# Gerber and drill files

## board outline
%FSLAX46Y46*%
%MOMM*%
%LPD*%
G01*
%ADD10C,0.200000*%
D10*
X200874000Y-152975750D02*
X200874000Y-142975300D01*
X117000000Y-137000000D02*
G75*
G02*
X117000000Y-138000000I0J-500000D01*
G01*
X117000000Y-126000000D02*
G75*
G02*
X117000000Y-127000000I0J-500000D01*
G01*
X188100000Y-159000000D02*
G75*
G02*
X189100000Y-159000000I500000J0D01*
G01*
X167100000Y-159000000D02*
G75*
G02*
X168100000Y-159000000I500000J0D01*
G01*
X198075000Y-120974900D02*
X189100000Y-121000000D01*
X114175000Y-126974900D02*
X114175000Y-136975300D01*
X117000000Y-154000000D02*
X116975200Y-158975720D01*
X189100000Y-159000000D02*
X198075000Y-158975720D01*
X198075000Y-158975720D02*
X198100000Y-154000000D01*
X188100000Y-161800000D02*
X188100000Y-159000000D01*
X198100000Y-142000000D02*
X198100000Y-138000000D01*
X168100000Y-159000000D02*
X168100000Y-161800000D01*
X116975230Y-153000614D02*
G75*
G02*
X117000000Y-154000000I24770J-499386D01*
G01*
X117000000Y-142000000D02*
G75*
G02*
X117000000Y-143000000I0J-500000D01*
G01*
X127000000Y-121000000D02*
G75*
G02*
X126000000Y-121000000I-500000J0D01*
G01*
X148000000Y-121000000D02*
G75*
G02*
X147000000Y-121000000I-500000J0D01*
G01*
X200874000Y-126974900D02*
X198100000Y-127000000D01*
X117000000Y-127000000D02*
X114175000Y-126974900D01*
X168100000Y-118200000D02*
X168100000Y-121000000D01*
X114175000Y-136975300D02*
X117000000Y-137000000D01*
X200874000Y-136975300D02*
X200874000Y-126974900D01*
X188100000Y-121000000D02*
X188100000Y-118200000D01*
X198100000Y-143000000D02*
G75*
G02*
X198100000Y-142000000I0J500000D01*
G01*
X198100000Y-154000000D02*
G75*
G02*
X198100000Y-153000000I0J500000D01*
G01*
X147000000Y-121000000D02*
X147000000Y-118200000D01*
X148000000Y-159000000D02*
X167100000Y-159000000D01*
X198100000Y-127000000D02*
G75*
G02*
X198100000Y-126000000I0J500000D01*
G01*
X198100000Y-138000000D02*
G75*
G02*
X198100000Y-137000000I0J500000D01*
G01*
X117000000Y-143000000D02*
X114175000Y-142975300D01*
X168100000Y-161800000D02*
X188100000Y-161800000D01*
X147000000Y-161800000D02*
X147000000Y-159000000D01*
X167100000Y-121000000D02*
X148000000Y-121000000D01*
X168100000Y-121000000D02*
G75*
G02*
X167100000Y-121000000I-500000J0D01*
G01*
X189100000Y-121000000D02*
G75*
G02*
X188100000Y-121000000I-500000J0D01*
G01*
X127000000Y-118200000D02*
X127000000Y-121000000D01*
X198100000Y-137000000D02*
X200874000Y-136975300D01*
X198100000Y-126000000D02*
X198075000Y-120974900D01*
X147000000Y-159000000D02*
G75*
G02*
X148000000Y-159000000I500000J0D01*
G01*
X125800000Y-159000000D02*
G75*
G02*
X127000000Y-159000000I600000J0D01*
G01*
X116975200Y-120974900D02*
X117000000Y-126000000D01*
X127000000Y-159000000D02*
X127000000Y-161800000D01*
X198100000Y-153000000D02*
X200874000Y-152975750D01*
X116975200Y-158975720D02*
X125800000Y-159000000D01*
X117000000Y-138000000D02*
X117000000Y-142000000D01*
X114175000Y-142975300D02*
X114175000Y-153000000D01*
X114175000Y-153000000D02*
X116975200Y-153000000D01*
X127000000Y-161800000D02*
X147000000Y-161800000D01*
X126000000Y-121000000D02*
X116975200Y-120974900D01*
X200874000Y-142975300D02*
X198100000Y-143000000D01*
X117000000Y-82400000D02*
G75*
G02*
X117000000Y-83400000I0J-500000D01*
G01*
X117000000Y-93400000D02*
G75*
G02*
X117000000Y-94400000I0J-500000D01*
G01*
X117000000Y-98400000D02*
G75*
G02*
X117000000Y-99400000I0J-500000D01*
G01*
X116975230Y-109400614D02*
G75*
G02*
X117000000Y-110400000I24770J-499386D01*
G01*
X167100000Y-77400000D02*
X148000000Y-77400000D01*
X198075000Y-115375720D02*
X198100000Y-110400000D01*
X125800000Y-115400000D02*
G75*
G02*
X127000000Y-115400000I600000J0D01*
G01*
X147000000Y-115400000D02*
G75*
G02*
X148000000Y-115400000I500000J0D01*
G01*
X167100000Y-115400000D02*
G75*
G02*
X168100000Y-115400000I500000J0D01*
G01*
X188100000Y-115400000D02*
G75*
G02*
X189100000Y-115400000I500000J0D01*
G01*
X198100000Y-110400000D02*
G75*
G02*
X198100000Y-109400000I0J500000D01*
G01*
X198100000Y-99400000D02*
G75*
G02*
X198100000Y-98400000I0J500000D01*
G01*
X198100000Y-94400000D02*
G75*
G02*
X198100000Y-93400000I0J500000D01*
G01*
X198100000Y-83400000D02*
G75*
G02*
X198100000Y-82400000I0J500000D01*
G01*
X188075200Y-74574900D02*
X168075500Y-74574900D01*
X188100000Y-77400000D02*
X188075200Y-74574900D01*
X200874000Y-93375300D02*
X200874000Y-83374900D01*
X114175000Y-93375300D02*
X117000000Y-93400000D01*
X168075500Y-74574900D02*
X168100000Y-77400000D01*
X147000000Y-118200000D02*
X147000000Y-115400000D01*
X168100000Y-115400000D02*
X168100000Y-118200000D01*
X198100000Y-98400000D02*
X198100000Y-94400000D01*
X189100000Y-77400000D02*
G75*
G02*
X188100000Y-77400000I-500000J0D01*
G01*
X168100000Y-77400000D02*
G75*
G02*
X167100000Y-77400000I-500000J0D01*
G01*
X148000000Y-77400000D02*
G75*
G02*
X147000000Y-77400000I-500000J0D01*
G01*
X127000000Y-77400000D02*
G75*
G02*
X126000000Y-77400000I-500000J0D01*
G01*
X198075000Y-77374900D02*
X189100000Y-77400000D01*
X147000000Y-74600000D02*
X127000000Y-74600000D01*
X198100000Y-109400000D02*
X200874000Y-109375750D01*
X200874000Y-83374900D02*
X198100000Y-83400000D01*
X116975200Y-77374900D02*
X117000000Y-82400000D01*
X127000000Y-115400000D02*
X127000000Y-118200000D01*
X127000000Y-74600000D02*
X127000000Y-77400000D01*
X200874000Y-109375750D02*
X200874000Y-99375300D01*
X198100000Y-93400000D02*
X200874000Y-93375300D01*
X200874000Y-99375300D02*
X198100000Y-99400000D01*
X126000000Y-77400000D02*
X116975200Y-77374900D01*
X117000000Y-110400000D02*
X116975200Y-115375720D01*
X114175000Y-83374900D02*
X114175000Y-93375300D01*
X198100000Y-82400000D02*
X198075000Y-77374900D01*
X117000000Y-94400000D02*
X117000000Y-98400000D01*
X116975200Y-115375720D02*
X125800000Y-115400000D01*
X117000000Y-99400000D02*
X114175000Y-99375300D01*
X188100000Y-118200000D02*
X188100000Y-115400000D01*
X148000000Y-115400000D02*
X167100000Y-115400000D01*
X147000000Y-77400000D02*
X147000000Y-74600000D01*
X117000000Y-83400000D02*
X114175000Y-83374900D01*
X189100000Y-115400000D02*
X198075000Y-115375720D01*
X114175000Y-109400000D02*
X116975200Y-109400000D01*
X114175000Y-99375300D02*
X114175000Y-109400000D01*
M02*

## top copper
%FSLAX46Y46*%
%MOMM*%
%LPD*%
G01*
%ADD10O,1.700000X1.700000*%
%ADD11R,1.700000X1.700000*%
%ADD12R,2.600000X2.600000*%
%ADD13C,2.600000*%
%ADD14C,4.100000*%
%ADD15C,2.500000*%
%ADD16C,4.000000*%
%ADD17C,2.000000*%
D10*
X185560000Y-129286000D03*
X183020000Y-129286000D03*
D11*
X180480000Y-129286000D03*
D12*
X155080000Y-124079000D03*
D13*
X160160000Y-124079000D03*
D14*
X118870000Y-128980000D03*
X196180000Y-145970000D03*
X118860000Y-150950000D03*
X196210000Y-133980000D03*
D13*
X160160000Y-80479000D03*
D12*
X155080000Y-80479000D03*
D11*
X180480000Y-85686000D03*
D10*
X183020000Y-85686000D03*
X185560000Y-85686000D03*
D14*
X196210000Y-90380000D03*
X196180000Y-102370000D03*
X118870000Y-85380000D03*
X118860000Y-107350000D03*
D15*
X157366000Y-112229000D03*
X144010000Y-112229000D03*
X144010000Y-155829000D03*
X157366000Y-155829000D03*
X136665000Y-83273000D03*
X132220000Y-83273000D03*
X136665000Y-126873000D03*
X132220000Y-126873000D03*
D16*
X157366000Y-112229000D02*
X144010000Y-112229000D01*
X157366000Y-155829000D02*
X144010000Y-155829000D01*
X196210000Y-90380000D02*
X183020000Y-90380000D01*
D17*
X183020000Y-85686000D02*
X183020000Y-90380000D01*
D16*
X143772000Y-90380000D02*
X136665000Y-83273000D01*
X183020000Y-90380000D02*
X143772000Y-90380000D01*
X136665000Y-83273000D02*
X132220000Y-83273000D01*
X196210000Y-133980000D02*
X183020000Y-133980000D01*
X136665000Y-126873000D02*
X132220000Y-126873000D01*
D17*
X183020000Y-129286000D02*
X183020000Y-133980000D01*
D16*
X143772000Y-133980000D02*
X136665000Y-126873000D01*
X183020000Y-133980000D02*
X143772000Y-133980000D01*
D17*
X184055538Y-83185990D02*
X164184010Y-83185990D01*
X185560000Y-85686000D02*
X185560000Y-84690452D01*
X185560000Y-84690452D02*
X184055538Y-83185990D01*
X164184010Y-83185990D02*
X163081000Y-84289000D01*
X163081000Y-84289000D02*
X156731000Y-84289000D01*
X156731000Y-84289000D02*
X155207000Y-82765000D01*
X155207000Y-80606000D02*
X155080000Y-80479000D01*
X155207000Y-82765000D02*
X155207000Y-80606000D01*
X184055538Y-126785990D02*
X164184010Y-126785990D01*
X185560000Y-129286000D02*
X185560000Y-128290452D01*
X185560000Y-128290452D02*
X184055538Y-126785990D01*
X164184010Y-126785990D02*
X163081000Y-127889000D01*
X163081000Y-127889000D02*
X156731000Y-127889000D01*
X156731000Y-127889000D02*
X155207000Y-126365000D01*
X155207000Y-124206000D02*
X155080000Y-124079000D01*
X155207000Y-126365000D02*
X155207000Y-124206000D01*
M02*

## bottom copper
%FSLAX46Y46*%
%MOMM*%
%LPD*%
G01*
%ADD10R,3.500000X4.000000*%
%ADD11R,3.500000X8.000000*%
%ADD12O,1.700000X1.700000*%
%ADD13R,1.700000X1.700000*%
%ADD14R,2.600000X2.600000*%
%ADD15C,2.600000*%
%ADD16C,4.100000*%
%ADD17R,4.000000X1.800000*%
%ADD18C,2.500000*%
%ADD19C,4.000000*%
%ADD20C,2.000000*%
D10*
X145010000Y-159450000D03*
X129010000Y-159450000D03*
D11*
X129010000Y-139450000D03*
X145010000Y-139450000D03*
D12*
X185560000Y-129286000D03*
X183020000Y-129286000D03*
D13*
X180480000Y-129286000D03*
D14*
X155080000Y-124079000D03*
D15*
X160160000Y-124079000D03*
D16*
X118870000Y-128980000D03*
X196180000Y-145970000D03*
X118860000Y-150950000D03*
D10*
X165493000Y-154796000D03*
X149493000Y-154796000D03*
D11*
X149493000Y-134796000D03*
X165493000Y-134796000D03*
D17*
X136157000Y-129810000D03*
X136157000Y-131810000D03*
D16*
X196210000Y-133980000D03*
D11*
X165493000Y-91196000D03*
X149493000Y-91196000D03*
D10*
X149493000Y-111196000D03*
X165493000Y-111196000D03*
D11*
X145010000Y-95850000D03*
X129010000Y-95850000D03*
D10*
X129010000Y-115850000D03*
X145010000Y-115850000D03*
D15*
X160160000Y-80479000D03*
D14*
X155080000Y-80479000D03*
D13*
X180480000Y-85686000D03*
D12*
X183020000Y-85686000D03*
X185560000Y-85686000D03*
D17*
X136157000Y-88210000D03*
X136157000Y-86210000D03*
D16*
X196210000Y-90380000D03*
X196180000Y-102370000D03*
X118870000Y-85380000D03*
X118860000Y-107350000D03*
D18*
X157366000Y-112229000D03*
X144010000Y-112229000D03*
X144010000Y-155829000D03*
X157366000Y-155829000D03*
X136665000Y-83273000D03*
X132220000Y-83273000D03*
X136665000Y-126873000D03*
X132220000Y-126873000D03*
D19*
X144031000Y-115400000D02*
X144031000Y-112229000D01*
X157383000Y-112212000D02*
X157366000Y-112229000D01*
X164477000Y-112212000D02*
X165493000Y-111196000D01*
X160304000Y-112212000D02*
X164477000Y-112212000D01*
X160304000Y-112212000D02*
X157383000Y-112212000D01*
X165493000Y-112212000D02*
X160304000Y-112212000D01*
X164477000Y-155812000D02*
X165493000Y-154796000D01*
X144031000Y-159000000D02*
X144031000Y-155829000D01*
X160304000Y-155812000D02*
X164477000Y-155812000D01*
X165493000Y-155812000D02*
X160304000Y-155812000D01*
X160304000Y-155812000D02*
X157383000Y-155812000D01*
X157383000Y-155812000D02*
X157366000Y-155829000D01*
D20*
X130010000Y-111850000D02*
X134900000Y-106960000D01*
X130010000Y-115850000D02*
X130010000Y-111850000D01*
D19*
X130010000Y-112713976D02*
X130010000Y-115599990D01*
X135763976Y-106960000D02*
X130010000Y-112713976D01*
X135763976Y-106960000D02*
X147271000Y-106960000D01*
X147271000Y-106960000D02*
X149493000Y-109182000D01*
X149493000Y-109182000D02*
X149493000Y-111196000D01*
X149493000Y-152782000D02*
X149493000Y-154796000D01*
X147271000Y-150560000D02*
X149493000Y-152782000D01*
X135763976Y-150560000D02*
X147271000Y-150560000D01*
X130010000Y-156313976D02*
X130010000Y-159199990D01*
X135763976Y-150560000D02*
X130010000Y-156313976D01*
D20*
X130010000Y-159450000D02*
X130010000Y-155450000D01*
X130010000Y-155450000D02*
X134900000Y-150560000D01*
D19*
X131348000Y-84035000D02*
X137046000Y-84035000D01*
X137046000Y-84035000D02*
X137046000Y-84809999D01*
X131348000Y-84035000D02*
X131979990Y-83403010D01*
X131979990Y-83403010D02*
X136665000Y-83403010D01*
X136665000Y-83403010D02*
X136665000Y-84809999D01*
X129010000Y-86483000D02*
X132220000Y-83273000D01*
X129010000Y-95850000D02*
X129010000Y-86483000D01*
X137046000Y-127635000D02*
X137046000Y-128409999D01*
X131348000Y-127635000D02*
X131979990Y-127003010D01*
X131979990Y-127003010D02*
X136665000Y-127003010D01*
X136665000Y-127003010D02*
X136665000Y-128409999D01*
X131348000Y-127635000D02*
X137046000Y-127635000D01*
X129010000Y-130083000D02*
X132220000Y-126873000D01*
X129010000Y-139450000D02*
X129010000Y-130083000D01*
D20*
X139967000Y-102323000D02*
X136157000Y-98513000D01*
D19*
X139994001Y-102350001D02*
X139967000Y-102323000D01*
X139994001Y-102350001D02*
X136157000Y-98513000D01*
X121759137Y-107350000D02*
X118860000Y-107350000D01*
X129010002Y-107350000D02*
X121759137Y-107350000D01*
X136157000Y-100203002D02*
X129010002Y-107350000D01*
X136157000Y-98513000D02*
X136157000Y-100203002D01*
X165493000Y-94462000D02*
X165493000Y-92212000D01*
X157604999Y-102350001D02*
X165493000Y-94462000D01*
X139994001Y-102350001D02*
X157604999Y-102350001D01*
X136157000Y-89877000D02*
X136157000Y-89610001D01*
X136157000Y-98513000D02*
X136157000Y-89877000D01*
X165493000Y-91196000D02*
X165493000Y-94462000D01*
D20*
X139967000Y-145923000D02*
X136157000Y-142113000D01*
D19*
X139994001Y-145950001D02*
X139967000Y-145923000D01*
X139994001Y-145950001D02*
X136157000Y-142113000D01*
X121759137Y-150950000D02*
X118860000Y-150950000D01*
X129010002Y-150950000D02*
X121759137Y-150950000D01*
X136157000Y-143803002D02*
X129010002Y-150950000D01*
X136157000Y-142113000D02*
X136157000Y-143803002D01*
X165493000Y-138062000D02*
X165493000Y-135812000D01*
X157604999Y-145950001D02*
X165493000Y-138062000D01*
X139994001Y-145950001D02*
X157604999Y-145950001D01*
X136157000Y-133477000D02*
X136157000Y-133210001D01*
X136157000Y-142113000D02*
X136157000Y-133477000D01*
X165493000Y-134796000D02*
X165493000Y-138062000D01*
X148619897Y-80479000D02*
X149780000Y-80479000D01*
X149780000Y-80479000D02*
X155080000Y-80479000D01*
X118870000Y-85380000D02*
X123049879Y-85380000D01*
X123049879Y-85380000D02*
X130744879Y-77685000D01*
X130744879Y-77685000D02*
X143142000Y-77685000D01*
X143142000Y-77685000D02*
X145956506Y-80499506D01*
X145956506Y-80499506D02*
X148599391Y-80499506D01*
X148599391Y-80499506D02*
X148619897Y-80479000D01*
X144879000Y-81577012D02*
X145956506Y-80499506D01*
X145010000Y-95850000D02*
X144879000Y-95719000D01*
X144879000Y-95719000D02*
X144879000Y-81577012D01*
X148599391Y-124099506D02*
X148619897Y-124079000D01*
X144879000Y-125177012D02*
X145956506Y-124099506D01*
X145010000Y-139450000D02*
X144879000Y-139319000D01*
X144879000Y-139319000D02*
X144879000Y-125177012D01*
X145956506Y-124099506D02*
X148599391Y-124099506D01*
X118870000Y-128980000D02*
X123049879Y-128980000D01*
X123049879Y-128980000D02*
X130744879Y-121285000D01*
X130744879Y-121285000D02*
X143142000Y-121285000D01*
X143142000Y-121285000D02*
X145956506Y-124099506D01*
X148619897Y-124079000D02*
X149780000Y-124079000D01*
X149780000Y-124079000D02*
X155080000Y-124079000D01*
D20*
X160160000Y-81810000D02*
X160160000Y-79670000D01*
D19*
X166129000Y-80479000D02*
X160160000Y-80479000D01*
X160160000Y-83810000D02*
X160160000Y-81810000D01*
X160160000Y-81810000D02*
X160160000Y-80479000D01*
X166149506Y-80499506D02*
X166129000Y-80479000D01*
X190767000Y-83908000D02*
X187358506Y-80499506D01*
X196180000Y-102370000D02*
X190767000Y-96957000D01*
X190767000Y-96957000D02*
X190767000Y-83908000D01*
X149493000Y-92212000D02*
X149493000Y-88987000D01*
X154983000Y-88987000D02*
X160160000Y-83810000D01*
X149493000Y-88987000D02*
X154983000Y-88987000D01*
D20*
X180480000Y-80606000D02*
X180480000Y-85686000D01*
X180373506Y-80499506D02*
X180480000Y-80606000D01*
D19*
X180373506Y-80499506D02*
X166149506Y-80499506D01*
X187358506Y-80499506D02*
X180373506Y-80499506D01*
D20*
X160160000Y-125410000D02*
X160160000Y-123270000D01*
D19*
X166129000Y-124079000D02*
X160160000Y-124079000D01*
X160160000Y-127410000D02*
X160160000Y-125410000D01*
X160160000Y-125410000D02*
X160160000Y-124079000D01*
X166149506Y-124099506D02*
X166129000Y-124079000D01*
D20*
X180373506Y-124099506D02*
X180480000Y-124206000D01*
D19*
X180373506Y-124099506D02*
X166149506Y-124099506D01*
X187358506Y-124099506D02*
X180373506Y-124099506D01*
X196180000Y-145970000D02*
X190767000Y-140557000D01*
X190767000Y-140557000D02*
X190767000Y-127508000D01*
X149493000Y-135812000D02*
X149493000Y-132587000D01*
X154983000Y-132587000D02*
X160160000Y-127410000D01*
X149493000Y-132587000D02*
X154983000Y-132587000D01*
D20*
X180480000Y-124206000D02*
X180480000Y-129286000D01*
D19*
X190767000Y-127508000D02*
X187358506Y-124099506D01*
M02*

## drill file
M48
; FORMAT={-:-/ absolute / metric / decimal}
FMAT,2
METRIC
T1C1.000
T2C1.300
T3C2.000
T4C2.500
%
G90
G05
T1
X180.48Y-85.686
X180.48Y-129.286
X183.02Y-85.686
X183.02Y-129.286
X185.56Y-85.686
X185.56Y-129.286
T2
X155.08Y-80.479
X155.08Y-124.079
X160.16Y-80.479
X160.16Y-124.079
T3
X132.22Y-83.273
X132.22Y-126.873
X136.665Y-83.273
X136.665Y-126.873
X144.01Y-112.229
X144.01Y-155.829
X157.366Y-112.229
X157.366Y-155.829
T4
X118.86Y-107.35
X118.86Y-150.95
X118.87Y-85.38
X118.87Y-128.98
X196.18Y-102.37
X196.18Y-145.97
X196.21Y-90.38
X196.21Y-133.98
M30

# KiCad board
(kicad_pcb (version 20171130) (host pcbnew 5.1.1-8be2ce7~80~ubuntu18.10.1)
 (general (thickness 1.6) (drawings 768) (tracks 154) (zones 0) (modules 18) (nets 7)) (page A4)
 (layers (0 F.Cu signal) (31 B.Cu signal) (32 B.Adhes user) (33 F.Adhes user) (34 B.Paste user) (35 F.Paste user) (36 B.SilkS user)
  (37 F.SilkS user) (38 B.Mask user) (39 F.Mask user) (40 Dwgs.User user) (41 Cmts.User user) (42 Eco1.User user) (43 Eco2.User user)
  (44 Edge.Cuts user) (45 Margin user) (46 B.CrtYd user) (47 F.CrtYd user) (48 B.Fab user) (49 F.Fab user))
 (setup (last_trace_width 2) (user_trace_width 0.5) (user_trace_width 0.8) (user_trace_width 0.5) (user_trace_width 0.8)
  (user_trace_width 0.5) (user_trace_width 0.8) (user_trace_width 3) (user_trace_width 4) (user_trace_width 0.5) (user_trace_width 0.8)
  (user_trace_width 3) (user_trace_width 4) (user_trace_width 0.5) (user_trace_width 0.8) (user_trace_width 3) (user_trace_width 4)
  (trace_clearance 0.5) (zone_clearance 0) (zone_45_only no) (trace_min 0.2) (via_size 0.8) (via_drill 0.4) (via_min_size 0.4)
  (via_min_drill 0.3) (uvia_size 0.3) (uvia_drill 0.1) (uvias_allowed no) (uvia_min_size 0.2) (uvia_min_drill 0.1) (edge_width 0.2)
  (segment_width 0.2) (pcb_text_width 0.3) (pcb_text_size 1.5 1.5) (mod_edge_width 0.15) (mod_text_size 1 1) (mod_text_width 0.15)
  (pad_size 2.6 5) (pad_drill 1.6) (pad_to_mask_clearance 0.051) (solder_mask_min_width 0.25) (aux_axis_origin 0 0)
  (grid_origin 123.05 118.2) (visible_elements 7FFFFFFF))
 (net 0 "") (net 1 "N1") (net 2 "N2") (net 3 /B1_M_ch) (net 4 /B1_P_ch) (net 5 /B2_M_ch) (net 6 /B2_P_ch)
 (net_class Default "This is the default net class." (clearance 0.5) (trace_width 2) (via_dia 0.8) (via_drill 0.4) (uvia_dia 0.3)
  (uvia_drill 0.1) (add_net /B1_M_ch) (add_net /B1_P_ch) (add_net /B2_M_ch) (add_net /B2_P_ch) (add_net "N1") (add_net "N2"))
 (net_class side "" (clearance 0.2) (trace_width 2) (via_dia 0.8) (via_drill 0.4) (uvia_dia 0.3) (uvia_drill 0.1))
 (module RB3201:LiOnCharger (layer B.Cu) (at 137.01 150.45)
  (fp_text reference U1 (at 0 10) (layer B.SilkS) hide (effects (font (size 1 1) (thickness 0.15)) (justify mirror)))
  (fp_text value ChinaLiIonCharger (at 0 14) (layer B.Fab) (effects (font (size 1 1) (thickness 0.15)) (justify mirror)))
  (pad 1 smd rect (at 8 9) (size 3.5 4) (layers B.Cu B.Paste B.Mask) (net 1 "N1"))
  (pad 2 smd rect (at -8 9) (size 3.5 4) (layers B.Cu B.Paste B.Mask) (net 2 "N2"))
  (pad 3 smd rect (at -8 -11) (size 3.5 8) (layers B.Cu B.Paste B.Mask) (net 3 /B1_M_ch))
  (pad 4 smd rect (at 8 -11) (size 3.5 8) (layers B.Cu B.Paste B.Mask) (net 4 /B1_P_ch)))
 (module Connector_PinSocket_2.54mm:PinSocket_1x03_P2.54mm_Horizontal (layer B.Cu) (at 180.48 129.286 270)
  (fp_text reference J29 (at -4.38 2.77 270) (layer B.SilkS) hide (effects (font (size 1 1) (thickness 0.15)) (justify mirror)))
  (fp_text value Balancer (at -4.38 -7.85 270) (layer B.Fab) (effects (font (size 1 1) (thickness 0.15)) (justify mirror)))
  (pad 3 thru_hole oval (at 0 -5.08 270) (size 1.7 1.7) (drill 1) (layers *.Cu *.Mask) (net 4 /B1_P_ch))
  (pad 2 thru_hole oval (at 0 -2.54 270) (size 1.7 1.7) (drill 1) (layers *.Cu *.Mask) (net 3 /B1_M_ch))
  (pad 1 thru_hole rect (at 0 0 270) (size 1.7 1.7) (drill 1) (layers *.Cu *.Mask) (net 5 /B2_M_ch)))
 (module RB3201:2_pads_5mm (layer B.Cu) (at 155.08 124.079)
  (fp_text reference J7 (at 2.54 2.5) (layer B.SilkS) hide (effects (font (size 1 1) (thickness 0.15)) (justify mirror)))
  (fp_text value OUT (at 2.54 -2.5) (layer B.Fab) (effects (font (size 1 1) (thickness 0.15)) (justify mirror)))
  (pad 1 thru_hole rect (at 0 0) (size 2.6 2.6) (drill 1.3) (layers *.Cu *.Mask) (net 4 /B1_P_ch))
  (pad 2 thru_hole circle (at 5.08 0) (size 2.6 2.6) (drill 1.3) (layers *.Cu *.Mask) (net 5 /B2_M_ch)))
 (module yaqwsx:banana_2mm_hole (layer F.Cu) (at 118.87 128.98)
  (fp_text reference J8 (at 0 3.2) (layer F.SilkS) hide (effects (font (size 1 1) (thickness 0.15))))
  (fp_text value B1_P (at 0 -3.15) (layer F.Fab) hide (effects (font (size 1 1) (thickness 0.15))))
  (pad 1 thru_hole circle (at 0 0) (size 4.1 4.1) (drill 2.5) (layers *.Cu *.Mask) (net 4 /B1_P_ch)))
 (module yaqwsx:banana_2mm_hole (layer F.Cu) (at 196.18 145.97)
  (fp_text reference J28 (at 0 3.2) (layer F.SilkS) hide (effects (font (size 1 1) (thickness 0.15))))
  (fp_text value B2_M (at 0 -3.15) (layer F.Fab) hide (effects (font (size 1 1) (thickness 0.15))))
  (pad 1 thru_hole circle (at 0 0) (size 4.1 4.1) (drill 2.5) (layers *.Cu *.Mask) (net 5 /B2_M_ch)))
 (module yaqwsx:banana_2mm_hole (layer F.Cu) (at 118.86 150.95)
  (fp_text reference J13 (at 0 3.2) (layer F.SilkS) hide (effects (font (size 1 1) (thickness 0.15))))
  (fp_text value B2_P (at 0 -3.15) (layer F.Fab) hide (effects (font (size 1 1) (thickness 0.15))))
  (pad 1 thru_hole circle (at 0 0) (size 4.1 4.1) (drill 2.5) (layers *.Cu *.Mask) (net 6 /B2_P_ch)))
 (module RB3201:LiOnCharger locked (layer B.Cu) (at 157.493 145.796)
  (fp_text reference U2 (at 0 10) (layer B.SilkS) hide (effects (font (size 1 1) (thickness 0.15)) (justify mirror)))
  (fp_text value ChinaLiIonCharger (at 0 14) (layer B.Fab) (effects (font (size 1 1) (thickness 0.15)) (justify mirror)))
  (pad 1 smd rect (at 8 9) (size 3.5 4) (layers B.Cu B.Paste B.Mask) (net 1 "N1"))
  (pad 2 smd rect (at -8 9) (size 3.5 4) (layers B.Cu B.Paste B.Mask) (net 2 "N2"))
  (pad 3 smd rect (at -8 -11) (size 3.5 8) (layers B.Cu B.Paste B.Mask) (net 5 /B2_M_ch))
  (pad 4 smd rect (at 8 -11) (size 3.5 8) (layers B.Cu B.Paste B.Mask) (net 6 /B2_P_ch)))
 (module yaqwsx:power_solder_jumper (layer B.Cu) (at 136.157 130.81 270)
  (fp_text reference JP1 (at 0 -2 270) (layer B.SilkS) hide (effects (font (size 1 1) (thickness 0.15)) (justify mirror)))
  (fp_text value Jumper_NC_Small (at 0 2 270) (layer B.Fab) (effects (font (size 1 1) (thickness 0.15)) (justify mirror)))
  (pad 1 smd rect (at -1 0 270) (size 1.8 4) (layers B.Cu B.Paste B.Mask) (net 3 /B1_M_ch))
  (pad 2 smd rect (at 1 0 270) (size 1.8 4) (layers B.Cu B.Paste B.Mask) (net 6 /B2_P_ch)))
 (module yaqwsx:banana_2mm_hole (layer F.Cu) (at 196.21 133.98)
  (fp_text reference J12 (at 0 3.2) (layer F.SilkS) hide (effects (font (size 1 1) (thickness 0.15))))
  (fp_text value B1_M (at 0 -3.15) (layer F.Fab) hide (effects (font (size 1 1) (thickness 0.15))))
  (pad 1 thru_hole circle (at 0 0) (size 4.1 4.1) (drill 2.5) (layers *.Cu *.Mask) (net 3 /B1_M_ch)))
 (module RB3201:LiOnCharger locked (layer B.Cu) (at 157.493 102.196)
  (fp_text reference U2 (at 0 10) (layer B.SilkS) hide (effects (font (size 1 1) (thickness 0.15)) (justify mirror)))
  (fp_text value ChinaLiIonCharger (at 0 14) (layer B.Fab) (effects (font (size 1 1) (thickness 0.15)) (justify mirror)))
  (pad 4 smd rect (at 8 -11) (size 3.5 8) (layers B.Cu B.Paste B.Mask) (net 6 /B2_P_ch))
  (pad 3 smd rect (at -8 -11) (size 3.5 8) (layers B.Cu B.Paste B.Mask) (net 5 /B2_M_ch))
  (pad 2 smd rect (at -8 9) (size 3.5 4) (layers B.Cu B.Paste B.Mask) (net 2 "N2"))
  (pad 1 smd rect (at 8 9) (size 3.5 4) (layers B.Cu B.Paste B.Mask) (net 1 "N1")))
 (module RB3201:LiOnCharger (layer B.Cu) (at 137.01 106.85)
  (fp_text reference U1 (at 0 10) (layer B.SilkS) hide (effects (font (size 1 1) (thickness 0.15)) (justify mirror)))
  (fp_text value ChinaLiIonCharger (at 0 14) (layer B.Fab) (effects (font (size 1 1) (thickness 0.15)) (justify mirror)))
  (pad 4 smd rect (at 8 -11) (size 3.5 8) (layers B.Cu B.Paste B.Mask) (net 4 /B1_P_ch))
  (pad 3 smd rect (at -8 -11) (size 3.5 8) (layers B.Cu B.Paste B.Mask) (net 3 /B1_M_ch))
  (pad 2 smd rect (at -8 9) (size 3.5 4) (layers B.Cu B.Paste B.Mask) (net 2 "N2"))
  (pad 1 smd rect (at 8 9) (size 3.5 4) (layers B.Cu B.Paste B.Mask) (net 1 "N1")))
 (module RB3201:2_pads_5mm (layer B.Cu) (at 155.08 80.479)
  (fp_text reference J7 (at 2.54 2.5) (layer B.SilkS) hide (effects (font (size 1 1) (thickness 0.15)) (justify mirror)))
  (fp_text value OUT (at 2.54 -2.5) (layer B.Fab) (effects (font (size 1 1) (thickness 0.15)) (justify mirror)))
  (pad 2 thru_hole circle (at 5.08 0) (size 2.6 2.6) (drill 1.3) (layers *.Cu *.Mask) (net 5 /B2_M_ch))
  (pad 1 thru_hole rect (at 0 0) (size 2.6 2.6) (drill 1.3) (layers *.Cu *.Mask) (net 4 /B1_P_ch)))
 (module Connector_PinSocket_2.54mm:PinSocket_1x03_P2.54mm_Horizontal (layer B.Cu) (at 180.48 85.686 270)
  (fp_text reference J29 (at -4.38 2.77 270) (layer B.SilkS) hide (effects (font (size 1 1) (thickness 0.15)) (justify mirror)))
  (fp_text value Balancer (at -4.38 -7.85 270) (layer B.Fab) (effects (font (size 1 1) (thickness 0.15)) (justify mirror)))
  (pad 1 thru_hole rect (at 0 0 270) (size 1.7 1.7) (drill 1) (layers *.Cu *.Mask) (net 5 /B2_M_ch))
  (pad 2 thru_hole oval (at 0 -2.54 270) (size 1.7 1.7) (drill 1) (layers *.Cu *.Mask) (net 3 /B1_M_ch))
  (pad 3 thru_hole oval (at 0 -5.08 270) (size 1.7 1.7) (drill 1) (layers *.Cu *.Mask) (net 4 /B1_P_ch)))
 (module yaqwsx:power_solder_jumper (layer B.Cu) (at 136.157 87.21 270)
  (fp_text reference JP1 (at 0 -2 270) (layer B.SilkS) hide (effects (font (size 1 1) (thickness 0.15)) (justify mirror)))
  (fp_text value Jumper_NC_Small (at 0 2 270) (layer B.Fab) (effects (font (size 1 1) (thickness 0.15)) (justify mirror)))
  (pad 2 smd rect (at 1 0 270) (size 1.8 4) (layers B.Cu B.Paste B.Mask) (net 6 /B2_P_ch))
  (pad 1 smd rect (at -1 0 270) (size 1.8 4) (layers B.Cu B.Paste B.Mask) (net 3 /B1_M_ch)))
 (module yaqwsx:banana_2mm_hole (layer F.Cu) (at 196.21 90.38)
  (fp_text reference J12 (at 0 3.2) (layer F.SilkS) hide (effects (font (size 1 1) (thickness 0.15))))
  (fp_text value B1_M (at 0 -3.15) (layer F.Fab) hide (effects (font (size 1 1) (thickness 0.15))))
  (pad 1 thru_hole circle (at 0 0) (size 4.1 4.1) (drill 2.5) (layers *.Cu *.Mask) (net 3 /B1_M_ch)))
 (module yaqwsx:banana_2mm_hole (layer F.Cu) (at 196.18 102.37)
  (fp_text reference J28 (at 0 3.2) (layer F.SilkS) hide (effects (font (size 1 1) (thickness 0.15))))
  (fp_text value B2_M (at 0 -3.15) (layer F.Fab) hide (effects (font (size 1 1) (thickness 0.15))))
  (pad 1 thru_hole circle (at 0 0) (size 4.1 4.1) (drill 2.5) (layers *.Cu *.Mask) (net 5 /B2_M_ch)))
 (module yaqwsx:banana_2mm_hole (layer F.Cu) (at 118.87 85.38)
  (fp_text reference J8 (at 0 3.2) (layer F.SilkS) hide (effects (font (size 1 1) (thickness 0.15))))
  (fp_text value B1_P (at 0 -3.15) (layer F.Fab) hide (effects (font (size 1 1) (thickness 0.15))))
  (pad 1 thru_hole circle (at 0 0) (size 4.1 4.1) (drill 2.5) (layers *.Cu *.Mask) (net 4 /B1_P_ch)))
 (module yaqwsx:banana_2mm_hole (layer F.Cu) (at 118.86 107.35)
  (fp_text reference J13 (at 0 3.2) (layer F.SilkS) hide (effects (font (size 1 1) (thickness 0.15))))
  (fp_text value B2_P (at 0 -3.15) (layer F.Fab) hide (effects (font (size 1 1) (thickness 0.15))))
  (pad 1 thru_hole circle (at 0 0) (size 4.1 4.1) (drill 2.5) (layers *.Cu *.Mask) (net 6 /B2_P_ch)))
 (gr_line (start 200.874 152.97575) (end 200.874 142.9753) (layer Edge.Cuts) (width 0.2))
 (gr_arc (start 117 137.5) (end 117 138) (angle -180) (layer Edge.Cuts) (width 0.2))
 (gr_arc (start 117 126.5) (end 117 127) (angle -180) (layer Edge.Cuts) (width 0.2))
 (gr_arc (start 188.6 159) (end 189.1 159) (angle -180) (layer Edge.Cuts) (width 0.2))
 (gr_arc (start 167.6 159) (end 168.1 159) (angle -180) (layer Edge.Cuts) (width 0.2))
 (gr_line (start 198.075 120.9749) (end 189.1 121) (layer Edge.Cuts) (width 0.2))
 (gr_line (start 114.175 126.9749) (end 114.175 136.9753) (layer Edge.Cuts) (width 0.2))
 (gr_line (start 117 154) (end 116.9752 158.97572) (layer Edge.Cuts) (width 0.2))
 (gr_line (start 189.1 159) (end 198.075 158.97572) (layer Edge.Cuts) (width 0.2))
 (gr_line (start 198.075 158.97572) (end 198.1 154) (layer Edge.Cuts) (width 0.2))
 (gr_line (start 188.1 161.8) (end 188.1 159) (layer Edge.Cuts) (width 0.2))
 (gr_line (start 198.1 142) (end 198.1 138) (layer Edge.Cuts) (width 0.2))
 (gr_line (start 168.1 159) (end 168.1 161.8) (layer Edge.Cuts) (width 0.2))
 (gr_arc (start 117 153.5) (end 117 154) (angle -182.8395436) (layer Edge.Cuts) (width 0.2))
 (gr_arc (start 117 142.5) (end 117 143) (angle -180) (layer Edge.Cuts) (width 0.2))
 (gr_arc (start 126.5 121) (end 126 121) (angle -180) (layer Edge.Cuts) (width 0.2))
 (gr_arc (start 147.5 121) (end 147 121) (angle -180) (layer Edge.Cuts) (width 0.2))
 (gr_line (start 200.874 126.9749) (end 198.1 127) (layer Edge.Cuts) (width 0.2))
 (gr_line (start 117 127) (end 114.175 126.9749) (layer Edge.Cuts) (width 0.2))
 (gr_line (start 168.1 118.2) (end 168.1 121) (layer Edge.Cuts) (width 0.2))
 (gr_line (start 114.175 136.9753) (end 117 137) (layer Edge.Cuts) (width 0.2))
 (gr_line (start 200.874 136.9753) (end 200.874 126.9749) (layer Edge.Cuts) (width 0.2))
 (gr_line (start 188.1 121) (end 188.1 118.2) (layer Edge.Cuts) (width 0.2))
 (gr_arc (start 198.1 142.5) (end 198.1 142) (angle -180) (layer Edge.Cuts) (width 0.2))
 (gr_arc (start 198.1 153.5) (end 198.1 153) (angle -180) (layer Edge.Cuts) (width 0.2))
 (gr_line (start 147 121) (end 147 118.2) (layer Edge.Cuts) (width 0.2))
 (gr_line (start 148 159) (end 167.1 159) (layer Edge.Cuts) (width 0.2))
 (gr_arc (start 198.1 126.5) (end 198.1 126) (angle -180) (layer Edge.Cuts) (width 0.2))
 (gr_arc (start 198.1 137.5) (end 198.1 137) (angle -180) (layer Edge.Cuts) (width 0.2))
 (gr_line (start 117 143) (end 114.175 142.9753) (layer Edge.Cuts) (width 0.2))
 (gr_line (start 168.1 161.8) (end 188.1 161.8) (layer Edge.Cuts) (width 0.2))
 (gr_line (start 147 161.8) (end 147 159) (layer Edge.Cuts) (width 0.2))
 (gr_line (start 167.1 121) (end 148 121) (layer Edge.Cuts) (width 0.2))
 (gr_arc (start 167.6 121) (end 167.1 121) (angle -180) (layer Edge.Cuts) (width 0.2))
 (gr_arc (start 188.6 121) (end 188.1 121) (angle -180) (layer Edge.Cuts) (width 0.2))
 (gr_line (start 127 118.2) (end 127 121) (layer Edge.Cuts) (width 0.2))
 (gr_line (start 198.1 137) (end 200.874 136.9753) (layer Edge.Cuts) (width 0.2))
 (gr_line (start 198.1 126) (end 198.075 120.9749) (layer Edge.Cuts) (width 0.2))
 (gr_arc (start 147.5 159) (end 148 159) (angle -180) (layer Edge.Cuts) (width 0.2))
 (gr_arc (start 126.4 159) (end 127 159) (angle -180) (layer Edge.Cuts) (width 0.2))
 (gr_line (start 116.9752 120.9749) (end 117 126) (layer Edge.Cuts) (width 0.2))
 (gr_line (start 127 159) (end 127 161.8) (layer Edge.Cuts) (width 0.2))
 (gr_line (start 198.1 153) (end 200.874 152.97575) (layer Edge.Cuts) (width 0.2))
 (gr_line (start 116.9752 158.97572) (end 125.8 159) (layer Edge.Cuts) (width 0.2))
 (gr_line (start 117 138) (end 117 142) (layer Edge.Cuts) (width 0.2))
 (gr_line (start 114.175 142.9753) (end 114.175 153) (layer Edge.Cuts) (width 0.2))
 (gr_line (start 114.175 153) (end 116.9752 153) (layer Edge.Cuts) (width 0.2))
 (gr_line (start 127 161.8) (end 147 161.8) (layer Edge.Cuts) (width 0.2))
 (gr_line (start 126 121) (end 116.9752 120.9749) (layer Edge.Cuts) (width 0.2))
 (gr_line (start 200.874 142.9753) (end 198.1 143) (layer Edge.Cuts) (width 0.2))
 (gr_arc (start 117 82.9) (end 117 83.4) (angle -180) (layer Edge.Cuts) (width 0.2))
 (gr_arc (start 117 93.9) (end 117 94.4) (angle -180) (layer Edge.Cuts) (width 0.2))
 (gr_arc (start 117 98.9) (end 117 99.4) (angle -180) (layer Edge.Cuts) (width 0.2))
 (gr_arc (start 117 109.9) (end 117 110.4) (angle -182.8395436) (layer Edge.Cuts) (width 0.2))
 (gr_line (start 167.1 77.4) (end 148 77.4) (layer Edge.Cuts) (width 0.2))
 (gr_line (start 198.075 115.37572) (end 198.1 110.4) (layer Edge.Cuts) (width 0.2))
 (gr_arc (start 126.4 115.4) (end 127 115.4) (angle -180) (layer Edge.Cuts) (width 0.2))
 (gr_arc (start 147.5 115.4) (end 148 115.4) (angle -180) (layer Edge.Cuts) (width 0.2))
 (gr_arc (start 167.6 115.4) (end 168.1 115.4) (angle -180) (layer Edge.Cuts) (width 0.2))
 (gr_arc (start 188.6 115.4) (end 189.1 115.4) (angle -180) (layer Edge.Cuts) (width 0.2))
 (gr_arc (start 198.1 109.9) (end 198.1 109.4) (angle -180) (layer Edge.Cuts) (width 0.2))
 (gr_arc (start 198.1 98.9) (end 198.1 98.4) (angle -180) (layer Edge.Cuts) (width 0.2))
 (gr_arc (start 198.1 93.9) (end 198.1 93.4) (angle -180) (layer Edge.Cuts) (width 0.2))
 (gr_arc (start 198.1 82.9) (end 198.1 82.4) (angle -180) (layer Edge.Cuts) (width 0.2))
 (gr_line (start 188.0752 74.5749) (end 168.0755 74.5749) (layer Edge.Cuts) (width 0.2))
 (gr_line (start 188.1 77.4) (end 188.0752 74.5749) (layer Edge.Cuts) (width 0.2))
 (gr_line (start 200.874 93.3753) (end 200.874 83.3749) (layer Edge.Cuts) (width 0.2))
 (gr_line (start 114.175 93.3753) (end 117 93.4) (layer Edge.Cuts) (width 0.2))
 (gr_line (start 168.0755 74.5749) (end 168.1 77.4) (layer Edge.Cuts) (width 0.2))
 (gr_line (start 147 118.2) (end 147 115.4) (layer Edge.Cuts) (width 0.2))
 (gr_line (start 168.1 115.4) (end 168.1 118.2) (layer Edge.Cuts) (width 0.2))
 (gr_line (start 198.1 98.4) (end 198.1 94.4) (layer Edge.Cuts) (width 0.2))
 (gr_arc (start 188.6 77.4) (end 188.1 77.4) (angle -180) (layer Edge.Cuts) (width 0.2))
 (gr_arc (start 167.6 77.4) (end 167.1 77.4) (angle -180) (layer Edge.Cuts) (width 0.2))
 (gr_arc (start 147.5 77.4) (end 147 77.4) (angle -180) (layer Edge.Cuts) (width 0.2))
 (gr_arc (start 126.5 77.4) (end 126 77.4) (angle -180) (layer Edge.Cuts) (width 0.2))
 (gr_line (start 198.075 77.3749) (end 189.1 77.4) (layer Edge.Cuts) (width 0.2))
 (gr_line (start 147 74.6) (end 127 74.6) (layer Edge.Cuts) (width 0.2))
 (gr_line (start 198.1 109.4) (end 200.874 109.37575) (layer Edge.Cuts) (width 0.2))
 (gr_line (start 200.874 83.3749) (end 198.1 83.4) (layer Edge.Cuts) (width 0.2))
 (gr_line (start 116.9752 77.3749) (end 117 82.4) (layer Edge.Cuts) (width 0.2))
 (gr_line (start 127 115.4) (end 127 118.2) (layer Edge.Cuts) (width 0.2))
 (gr_line (start 127 74.6) (end 127 77.4) (layer Edge.Cuts) (width 0.2))
 (gr_line (start 200.874 109.37575) (end 200.874 99.3753) (layer Edge.Cuts) (width 0.2))
 (gr_line (start 198.1 93.4) (end 200.874 93.3753) (layer Edge.Cuts) (width 0.2))
 (gr_line (start 200.874 99.3753) (end 198.1 99.4) (layer Edge.Cuts) (width 0.2))
 (gr_line (start 126 77.4) (end 116.9752 77.3749) (layer Edge.Cuts) (width 0.2))
 (gr_line (start 117 110.4) (end 116.9752 115.37572) (layer Edge.Cuts) (width 0.2))
 (gr_line (start 114.175 83.3749) (end 114.175 93.3753) (layer Edge.Cuts) (width 0.2))
 (gr_line (start 198.1 82.4) (end 198.075 77.3749) (layer Edge.Cuts) (width 0.2))
 (gr_line (start 117 94.4) (end 117 98.4) (layer Edge.Cuts) (width 0.2))
 (gr_line (start 116.9752 115.37572) (end 125.8 115.4) (layer Edge.Cuts) (width 0.2))
 (gr_line (start 117 99.4) (end 114.175 99.3753) (layer Edge.Cuts) (width 0.2))
 (gr_line (start 188.1 118.2) (end 188.1 115.4) (layer Edge.Cuts) (width 0.2))
 (gr_line (start 148 115.4) (end 167.1 115.4) (layer Edge.Cuts) (width 0.2))
 (gr_line (start 147 77.4) (end 147 74.6) (layer Edge.Cuts) (width 0.2))
 (gr_line (start 117 83.4) (end 114.175 83.3749) (layer Edge.Cuts) (width 0.2))
 (gr_line (start 189.1 115.4) (end 198.075 115.37572) (layer Edge.Cuts) (width 0.2))
 (gr_line (start 114.175 109.4) (end 116.9752 109.4) (layer Edge.Cuts) (width 0.2))
 (gr_line (start 114.175 99.3753) (end 114.175 109.4) (layer Edge.Cuts) (width 0.2))
 (segment (start 144.031 115.4) (end 144.031 112.229) (width 4) (layer B.Cu) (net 1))
 (via (at 157.366 112.229) (size 2.5) (drill 2) (layers F.Cu B.Cu) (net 1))
 (segment (start 157.383 112.212) (end 157.366 112.229) (width 4) (layer B.Cu) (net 1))
 (via (at 144.01 112.229) (size 2.5) (drill 2) (layers F.Cu B.Cu) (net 1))
 (segment (start 157.366 112.229) (end 144.01 112.229) (width 4) (layer F.Cu) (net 1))
 (segment (start 164.477 112.212) (end 165.493 111.196) (width 4) (layer B.Cu) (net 1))
 (segment (start 160.304 112.212) (end 164.477 112.212) (width 4) (layer B.Cu) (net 1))
 (segment (start 160.304 112.212) (end 157.383 112.212) (width 4) (layer B.Cu) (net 1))
 (segment (start 165.493 112.212) (end 160.304 112.212) (width 4) (layer B.Cu) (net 1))
 (segment (start 157.366 155.829) (end 144.01 155.829) (width 4) (layer F.Cu) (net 1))
 (segment (start 164.477 155.812) (end 165.493 154.796) (width 4) (layer B.Cu) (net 1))
 (segment (start 144.031 159) (end 144.031 155.829) (width 4) (layer B.Cu) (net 1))
 (via (at 144.01 155.829) (size 2.5) (drill 2) (layers F.Cu B.Cu) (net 1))
 (via (at 157.366 155.829) (size 2.5) (drill 2) (layers F.Cu B.Cu) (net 1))
 (segment (start 160.304 155.812) (end 164.477 155.812) (width 4) (layer B.Cu) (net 1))
 (segment (start 165.493 155.812) (end 160.304 155.812) (width 4) (layer B.Cu) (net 1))
 (segment (start 160.304 155.812) (end 157.383 155.812) (width 4) (layer B.Cu) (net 1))
 (segment (start 157.383 155.812) (end 157.366 155.829) (width 4) (layer B.Cu) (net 1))
 (segment (start 130.01 111.85) (end 134.9 106.96) (width 2) (layer B.Cu) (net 2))
 (segment (start 130.01 115.85) (end 130.01 111.85) (width 2) (layer B.Cu) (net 2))
 (segment (start 130.01 112.713976) (end 130.01 115.59999) (width 4) (layer B.Cu) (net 2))
 (segment (start 135.763976 106.96) (end 130.01 112.713976) (width 4) (layer B.Cu) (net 2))
 (segment (start 135.763976 106.96) (end 147.271 106.96) (width 4) (layer B.Cu) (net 2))
 (segment (start 147.271 106.96) (end 149.493 109.182) (width 4) (layer B.Cu) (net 2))
 (segment (start 149.493 109.182) (end 149.493 111.196) (width 4) (layer B.Cu) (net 2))
 (segment (start 149.493 152.782) (end 149.493 154.796) (width 4) (layer B.Cu) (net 2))
 (segment (start 147.271 150.56) (end 149.493 152.782) (width 4) (layer B.Cu) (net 2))
 (segment (start 135.763976 150.56) (end 147.271 150.56) (width 4) (layer B.Cu) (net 2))
 (segment (start 130.01 156.313976) (end 130.01 159.19999) (width 4) (layer B.Cu) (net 2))
 (segment (start 135.763976 150.56) (end 130.01 156.313976) (width 4) (layer B.Cu) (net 2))
 (segment (start 130.01 159.45) (end 130.01 155.45) (width 2) (layer B.Cu) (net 2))
 (segment (start 130.01 155.45) (end 134.9 150.56) (width 2) (layer B.Cu) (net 2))
 (segment (start 131.348 84.035) (end 137.046 84.035) (width 4) (layer B.Cu) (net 3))
 (segment (start 137.046 84.035) (end 137.046 84.809999) (width 4) (layer B.Cu) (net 3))
 (via (at 136.665 83.273) (size 2.5) (drill 2) (layers F.Cu B.Cu) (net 3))
 (via (at 132.22 83.273) (size 2.5) (drill 2) (layers F.Cu B.Cu) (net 3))
 (segment (start 131.348 84.035) (end 131.97999 83.40301) (width 4) (layer B.Cu) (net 3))
 (segment (start 131.97999 83.40301) (end 136.665 83.40301) (width 4) (layer B.Cu) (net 3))
 (segment (start 136.665 83.40301) (end 136.665 84.809999) (width 4) (layer B.Cu) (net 3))
 (segment (start 196.21 90.38) (end 183.02 90.38) (width 4) (layer F.Cu) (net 3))
 (segment (start 183.02 85.686) (end 183.02 90.38) (width 2) (layer F.Cu) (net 3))
 (segment (start 129.01 86.483) (end 132.22 83.273) (width 4) (layer B.Cu) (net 3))
 (segment (start 129.01 95.85) (end 129.01 86.483) (width 4) (layer B.Cu) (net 3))
 (segment (start 143.772 90.38) (end 136.665 83.273) (width 4) (layer F.Cu) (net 3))
 (segment (start 183.02 90.38) (end 143.772 90.38) (width 4) (layer F.Cu) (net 3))
 (segment (start 136.665 83.273) (end 132.22 83.273) (width 4) (layer F.Cu) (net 3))
 (segment (start 137.046 127.635) (end 137.046 128.409999) (width 4) (layer B.Cu) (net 3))
 (via (at 136.665 126.873) (size 2.5) (drill 2) (layers F.Cu B.Cu) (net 3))
 (segment (start 131.348 127.635) (end 131.97999 127.00301) (width 4) (layer B.Cu) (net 3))
 (segment (start 131.97999 127.00301) (end 136.665 127.00301) (width 4) (layer B.Cu) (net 3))
 (segment (start 136.665 127.00301) (end 136.665 128.409999) (width 4) (layer B.Cu) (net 3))
 (segment (start 196.21 133.98) (end 183.02 133.98) (width 4) (layer F.Cu) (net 3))
 (segment (start 136.665 126.873) (end 132.22 126.873) (width 4) (layer F.Cu) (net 3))
 (segment (start 131.348 127.635) (end 137.046 127.635) (width 4) (layer B.Cu) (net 3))
 (via (at 132.22 126.873) (size 2.5) (drill 2) (layers F.Cu B.Cu) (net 3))
 (segment (start 183.02 129.286) (end 183.02 133.98) (width 2) (layer F.Cu) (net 3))
 (segment (start 129.01 130.083) (end 132.22 126.873) (width 4) (layer B.Cu) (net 3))
 (segment (start 129.01 139.45) (end 129.01 130.083) (width 4) (layer B.Cu) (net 3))
 (segment (start 143.772 133.98) (end 136.665 126.873) (width 4) (layer F.Cu) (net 3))
 (segment (start 183.02 133.98) (end 143.772 133.98) (width 4) (layer F.Cu) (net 3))
 (segment (start 139.967 102.323) (end 136.157 98.513) (width 2) (layer B.Cu) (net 6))
 (segment (start 139.994001 102.350001) (end 139.967 102.323) (width 4) (layer B.Cu) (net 6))
 (segment (start 139.994001 102.350001) (end 136.157 98.513) (width 4) (layer B.Cu) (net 6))
 (segment (start 121.759137 107.35) (end 118.86 107.35) (width 4) (layer B.Cu) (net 6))
 (segment (start 129.010002 107.35) (end 121.759137 107.35) (width 4) (layer B.Cu) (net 6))
 (segment (start 136.157 100.203002) (end 129.010002 107.35) (width 4) (layer B.Cu) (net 6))
 (segment (start 136.157 98.513) (end 136.157 100.203002) (width 4) (layer B.Cu) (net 6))
 (segment (start 165.493 94.462) (end 165.493 92.212) (width 4) (layer B.Cu) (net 6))
 (segment (start 157.604999 102.350001) (end 165.493 94.462) (width 4) (layer B.Cu) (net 6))
 (segment (start 139.994001 102.350001) (end 157.604999 102.350001) (width 4) (layer B.Cu) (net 6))
 (segment (start 136.157 89.877) (end 136.157 89.610001) (width 4) (layer B.Cu) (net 6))
 (segment (start 136.157 98.513) (end 136.157 89.877) (width 4) (layer B.Cu) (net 6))
 (segment (start 165.493 91.196) (end 165.493 94.462) (width 4) (layer B.Cu) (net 6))
 (segment (start 139.967 145.923) (end 136.157 142.113) (width 2) (layer B.Cu) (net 6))
 (segment (start 139.994001 145.950001) (end 139.967 145.923) (width 4) (layer B.Cu) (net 6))
 (segment (start 139.994001 145.950001) (end 136.157 142.113) (width 4) (layer B.Cu) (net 6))
 (segment (start 121.759137 150.95) (end 118.86 150.95) (width 4) (layer B.Cu) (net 6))
 (segment (start 129.010002 150.95) (end 121.759137 150.95) (width 4) (layer B.Cu) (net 6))
 (segment (start 136.157 143.803002) (end 129.010002 150.95) (width 4) (layer B.Cu) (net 6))
 (segment (start 136.157 142.113) (end 136.157 143.803002) (width 4) (layer B.Cu) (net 6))
 (segment (start 165.493 138.062) (end 165.493 135.812) (width 4) (layer B.Cu) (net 6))
 (segment (start 157.604999 145.950001) (end 165.493 138.062) (width 4) (layer B.Cu) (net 6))
 (segment (start 139.994001 145.950001) (end 157.604999 145.950001) (width 4) (layer B.Cu) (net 6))
 (segment (start 136.157 133.477) (end 136.157 133.210001) (width 4) (layer B.Cu) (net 6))
 (segment (start 136.157 142.113) (end 136.157 133.477) (width 4) (layer B.Cu) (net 6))
 (segment (start 165.493 134.796) (end 165.493 138.062) (width 4) (layer B.Cu) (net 6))
 (segment (start 184.055538 83.18599) (end 164.18401 83.18599) (width 2) (layer F.Cu) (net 4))
 (segment (start 185.56 85.686) (end 185.56 84.690452) (width 2) (layer F.Cu) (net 4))
 (segment (start 185.56 84.690452) (end 184.055538 83.18599) (width 2) (layer F.Cu) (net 4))
 (segment (start 164.18401 83.18599) (end 163.081 84.289) (width 2) (layer F.Cu) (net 4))
 (segment (start 163.081 84.289) (end 156.731 84.289) (width 2) (layer F.Cu) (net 4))
 (segment (start 156.731 84.289) (end 155.207 82.765) (width 2) (layer F.Cu) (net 4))
 (segment (start 155.207 80.606) (end 155.08 80.479) (width 2) (layer F.Cu) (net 4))
 (segment (start 155.207 82.765) (end 155.207 80.606) (width 2) (layer F.Cu) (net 4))
 (segment (start 148.619897 80.479) (end 149.78 80.479) (width 4) (layer B.Cu) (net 4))
 (segment (start 149.78 80.479) (end 155.08 80.479) (width 4) (layer B.Cu) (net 4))
 (segment (start 118.87 85.38) (end 123.049879 85.38) (width 4) (layer B.Cu) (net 4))
 (segment (start 123.049879 85.38) (end 130.744879 77.685) (width 4) (layer B.Cu) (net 4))
 (segment (start 130.744879 77.685) (end 143.142 77.685) (width 4) (layer B.Cu) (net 4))
 (segment (start 143.142 77.685) (end 145.956506 80.499506) (width 4) (layer B.Cu) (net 4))
 (segment (start 145.956506 80.499506) (end 148.599391 80.499506) (width 4) (layer B.Cu) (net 4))
 (segment (start 148.599391 80.499506) (end 148.619897 80.479) (width 4) (layer B.Cu) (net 4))
 (segment (start 144.879 81.577012) (end 145.956506 80.499506) (width 4) (layer B.Cu) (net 4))
 (segment (start 145.01 95.85) (end 144.879 95.719) (width 4) (layer B.Cu) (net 4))
 (segment (start 144.879 95.719) (end 144.879 81.577012) (width 4) (layer B.Cu) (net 4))
 (segment (start 148.599391 124.099506) (end 148.619897 124.079) (width 4) (layer B.Cu) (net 4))
 (segment (start 144.879 125.177012) (end 145.956506 124.099506) (width 4) (layer B.Cu) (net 4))
 (segment (start 145.01 139.45) (end 144.879 139.319) (width 4) (layer B.Cu) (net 4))
 (segment (start 144.879 139.319) (end 144.879 125.177012) (width 4) (layer B.Cu) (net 4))
 (segment (start 145.956506 124.099506) (end 148.599391 124.099506) (width 4) (layer B.Cu) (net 4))
 (segment (start 184.055538 126.78599) (end 164.18401 126.78599) (width 2) (layer F.Cu) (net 4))
 (segment (start 118.87 128.98) (end 123.049879 128.98) (width 4) (layer B.Cu) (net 4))
 (segment (start 123.049879 128.98) (end 130.744879 121.285) (width 4) (layer B.Cu) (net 4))
 (segment (start 130.744879 121.285) (end 143.142 121.285) (width 4) (layer B.Cu) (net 4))
 (segment (start 143.142 121.285) (end 145.956506 124.099506) (width 4) (layer B.Cu) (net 4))
 (segment (start 185.56 129.286) (end 185.56 128.290452) (width 2) (layer F.Cu) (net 4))
 (segment (start 185.56 128.290452) (end 184.055538 126.78599) (width 2) (layer F.Cu) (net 4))
 (segment (start 164.18401 126.78599) (end 163.081 127.889) (width 2) (layer F.Cu) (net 4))
 (segment (start 163.081 127.889) (end 156.731 127.889) (width 2) (layer F.Cu) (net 4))
 (segment (start 156.731 127.889) (end 155.207 126.365) (width 2) (layer F.Cu) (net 4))
 (segment (start 155.207 124.206) (end 155.08 124.079) (width 2) (layer F.Cu) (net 4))
 (segment (start 155.207 126.365) (end 155.207 124.206) (width 2) (layer F.Cu) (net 4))
 (segment (start 148.619897 124.079) (end 149.78 124.079) (width 4) (layer B.Cu) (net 4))
 (segment (start 149.78 124.079) (end 155.08 124.079) (width 4) (layer B.Cu) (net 4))
 (segment (start 160.16 81.81) (end 160.16 79.67) (width 2) (layer B.Cu) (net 5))
 (segment (start 166.129 80.479) (end 160.16 80.479) (width 4) (layer B.Cu) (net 5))
 (segment (start 160.16 83.81) (end 160.16 81.81) (width 4) (layer B.Cu) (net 5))
 (segment (start 160.16 81.81) (end 160.16 80.479) (width 4) (layer B.Cu) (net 5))
 (segment (start 166.149506 80.499506) (end 166.129 80.479) (width 4) (layer B.Cu) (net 5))
 (segment (start 190.767 83.908) (end 187.358506 80.499506) (width 4) (layer B.Cu) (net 5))
 (segment (start 196.18 102.37) (end 190.767 96.957) (width 4) (layer B.Cu) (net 5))
 (segment (start 190.767 96.957) (end 190.767 83.908) (width 4) (layer B.Cu) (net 5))
 (segment (start 149.493 92.212) (end 149.493 88.987) (width 4) (layer B.Cu) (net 5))
 (segment (start 154.983 88.987) (end 160.16 83.81) (width 4) (layer B.Cu) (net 5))
 (segment (start 149.493 88.987) (end 154.983 88.987) (width 4) (layer B.Cu) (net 5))
 (segment (start 180.48 80.606) (end 180.48 85.686) (width 2) (layer B.Cu) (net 5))
 (segment (start 180.373506 80.499506) (end 180.48 80.606) (width 2) (layer B.Cu) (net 5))
 (segment (start 180.373506 80.499506) (end 166.149506 80.499506) (width 4) (layer B.Cu) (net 5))
 (segment (start 187.358506 80.499506) (end 180.373506 80.499506) (width 4) (layer B.Cu) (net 5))
 (segment (start 160.16 125.41) (end 160.16 123.27) (width 2) (layer B.Cu) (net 5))
 (segment (start 166.129 124.079) (end 160.16 124.079) (width 4) (layer B.Cu) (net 5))
 (segment (start 160.16 127.41) (end 160.16 125.41) (width 4) (layer B.Cu) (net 5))
 (segment (start 160.16 125.41) (end 160.16 124.079) (width 4) (layer B.Cu) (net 5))
 (segment (start 166.149506 124.099506) (end 166.129 124.079) (width 4) (layer B.Cu) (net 5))
 (segment (start 180.373506 124.099506) (end 180.48 124.206) (width 2) (layer B.Cu) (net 5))
 (segment (start 180.373506 124.099506) (end 166.149506 124.099506) (width 4) (layer B.Cu) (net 5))
 (segment (start 187.358506 124.099506) (end 180.373506 124.099506) (width 4) (layer B.Cu) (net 5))
 (segment (start 196.18 145.97) (end 190.767 140.557) (width 4) (layer B.Cu) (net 5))
 (segment (start 190.767 140.557) (end 190.767 127.508) (width 4) (layer B.Cu) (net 5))
 (segment (start 149.493 135.812) (end 149.493 132.587) (width 4) (layer B.Cu) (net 5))
 (segment (start 154.983 132.587) (end 160.16 127.41) (width 4) (layer B.Cu) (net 5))
 (segment (start 149.493 132.587) (end 154.983 132.587) (width 4) (layer B.Cu) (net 5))
 (segment (start 180.48 124.206) (end 180.48 129.286) (width 2) (layer B.Cu) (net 5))
 (segment (start 190.767 127.508) (end 187.358506 124.099506) (width 4) (layer B.Cu) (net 5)))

